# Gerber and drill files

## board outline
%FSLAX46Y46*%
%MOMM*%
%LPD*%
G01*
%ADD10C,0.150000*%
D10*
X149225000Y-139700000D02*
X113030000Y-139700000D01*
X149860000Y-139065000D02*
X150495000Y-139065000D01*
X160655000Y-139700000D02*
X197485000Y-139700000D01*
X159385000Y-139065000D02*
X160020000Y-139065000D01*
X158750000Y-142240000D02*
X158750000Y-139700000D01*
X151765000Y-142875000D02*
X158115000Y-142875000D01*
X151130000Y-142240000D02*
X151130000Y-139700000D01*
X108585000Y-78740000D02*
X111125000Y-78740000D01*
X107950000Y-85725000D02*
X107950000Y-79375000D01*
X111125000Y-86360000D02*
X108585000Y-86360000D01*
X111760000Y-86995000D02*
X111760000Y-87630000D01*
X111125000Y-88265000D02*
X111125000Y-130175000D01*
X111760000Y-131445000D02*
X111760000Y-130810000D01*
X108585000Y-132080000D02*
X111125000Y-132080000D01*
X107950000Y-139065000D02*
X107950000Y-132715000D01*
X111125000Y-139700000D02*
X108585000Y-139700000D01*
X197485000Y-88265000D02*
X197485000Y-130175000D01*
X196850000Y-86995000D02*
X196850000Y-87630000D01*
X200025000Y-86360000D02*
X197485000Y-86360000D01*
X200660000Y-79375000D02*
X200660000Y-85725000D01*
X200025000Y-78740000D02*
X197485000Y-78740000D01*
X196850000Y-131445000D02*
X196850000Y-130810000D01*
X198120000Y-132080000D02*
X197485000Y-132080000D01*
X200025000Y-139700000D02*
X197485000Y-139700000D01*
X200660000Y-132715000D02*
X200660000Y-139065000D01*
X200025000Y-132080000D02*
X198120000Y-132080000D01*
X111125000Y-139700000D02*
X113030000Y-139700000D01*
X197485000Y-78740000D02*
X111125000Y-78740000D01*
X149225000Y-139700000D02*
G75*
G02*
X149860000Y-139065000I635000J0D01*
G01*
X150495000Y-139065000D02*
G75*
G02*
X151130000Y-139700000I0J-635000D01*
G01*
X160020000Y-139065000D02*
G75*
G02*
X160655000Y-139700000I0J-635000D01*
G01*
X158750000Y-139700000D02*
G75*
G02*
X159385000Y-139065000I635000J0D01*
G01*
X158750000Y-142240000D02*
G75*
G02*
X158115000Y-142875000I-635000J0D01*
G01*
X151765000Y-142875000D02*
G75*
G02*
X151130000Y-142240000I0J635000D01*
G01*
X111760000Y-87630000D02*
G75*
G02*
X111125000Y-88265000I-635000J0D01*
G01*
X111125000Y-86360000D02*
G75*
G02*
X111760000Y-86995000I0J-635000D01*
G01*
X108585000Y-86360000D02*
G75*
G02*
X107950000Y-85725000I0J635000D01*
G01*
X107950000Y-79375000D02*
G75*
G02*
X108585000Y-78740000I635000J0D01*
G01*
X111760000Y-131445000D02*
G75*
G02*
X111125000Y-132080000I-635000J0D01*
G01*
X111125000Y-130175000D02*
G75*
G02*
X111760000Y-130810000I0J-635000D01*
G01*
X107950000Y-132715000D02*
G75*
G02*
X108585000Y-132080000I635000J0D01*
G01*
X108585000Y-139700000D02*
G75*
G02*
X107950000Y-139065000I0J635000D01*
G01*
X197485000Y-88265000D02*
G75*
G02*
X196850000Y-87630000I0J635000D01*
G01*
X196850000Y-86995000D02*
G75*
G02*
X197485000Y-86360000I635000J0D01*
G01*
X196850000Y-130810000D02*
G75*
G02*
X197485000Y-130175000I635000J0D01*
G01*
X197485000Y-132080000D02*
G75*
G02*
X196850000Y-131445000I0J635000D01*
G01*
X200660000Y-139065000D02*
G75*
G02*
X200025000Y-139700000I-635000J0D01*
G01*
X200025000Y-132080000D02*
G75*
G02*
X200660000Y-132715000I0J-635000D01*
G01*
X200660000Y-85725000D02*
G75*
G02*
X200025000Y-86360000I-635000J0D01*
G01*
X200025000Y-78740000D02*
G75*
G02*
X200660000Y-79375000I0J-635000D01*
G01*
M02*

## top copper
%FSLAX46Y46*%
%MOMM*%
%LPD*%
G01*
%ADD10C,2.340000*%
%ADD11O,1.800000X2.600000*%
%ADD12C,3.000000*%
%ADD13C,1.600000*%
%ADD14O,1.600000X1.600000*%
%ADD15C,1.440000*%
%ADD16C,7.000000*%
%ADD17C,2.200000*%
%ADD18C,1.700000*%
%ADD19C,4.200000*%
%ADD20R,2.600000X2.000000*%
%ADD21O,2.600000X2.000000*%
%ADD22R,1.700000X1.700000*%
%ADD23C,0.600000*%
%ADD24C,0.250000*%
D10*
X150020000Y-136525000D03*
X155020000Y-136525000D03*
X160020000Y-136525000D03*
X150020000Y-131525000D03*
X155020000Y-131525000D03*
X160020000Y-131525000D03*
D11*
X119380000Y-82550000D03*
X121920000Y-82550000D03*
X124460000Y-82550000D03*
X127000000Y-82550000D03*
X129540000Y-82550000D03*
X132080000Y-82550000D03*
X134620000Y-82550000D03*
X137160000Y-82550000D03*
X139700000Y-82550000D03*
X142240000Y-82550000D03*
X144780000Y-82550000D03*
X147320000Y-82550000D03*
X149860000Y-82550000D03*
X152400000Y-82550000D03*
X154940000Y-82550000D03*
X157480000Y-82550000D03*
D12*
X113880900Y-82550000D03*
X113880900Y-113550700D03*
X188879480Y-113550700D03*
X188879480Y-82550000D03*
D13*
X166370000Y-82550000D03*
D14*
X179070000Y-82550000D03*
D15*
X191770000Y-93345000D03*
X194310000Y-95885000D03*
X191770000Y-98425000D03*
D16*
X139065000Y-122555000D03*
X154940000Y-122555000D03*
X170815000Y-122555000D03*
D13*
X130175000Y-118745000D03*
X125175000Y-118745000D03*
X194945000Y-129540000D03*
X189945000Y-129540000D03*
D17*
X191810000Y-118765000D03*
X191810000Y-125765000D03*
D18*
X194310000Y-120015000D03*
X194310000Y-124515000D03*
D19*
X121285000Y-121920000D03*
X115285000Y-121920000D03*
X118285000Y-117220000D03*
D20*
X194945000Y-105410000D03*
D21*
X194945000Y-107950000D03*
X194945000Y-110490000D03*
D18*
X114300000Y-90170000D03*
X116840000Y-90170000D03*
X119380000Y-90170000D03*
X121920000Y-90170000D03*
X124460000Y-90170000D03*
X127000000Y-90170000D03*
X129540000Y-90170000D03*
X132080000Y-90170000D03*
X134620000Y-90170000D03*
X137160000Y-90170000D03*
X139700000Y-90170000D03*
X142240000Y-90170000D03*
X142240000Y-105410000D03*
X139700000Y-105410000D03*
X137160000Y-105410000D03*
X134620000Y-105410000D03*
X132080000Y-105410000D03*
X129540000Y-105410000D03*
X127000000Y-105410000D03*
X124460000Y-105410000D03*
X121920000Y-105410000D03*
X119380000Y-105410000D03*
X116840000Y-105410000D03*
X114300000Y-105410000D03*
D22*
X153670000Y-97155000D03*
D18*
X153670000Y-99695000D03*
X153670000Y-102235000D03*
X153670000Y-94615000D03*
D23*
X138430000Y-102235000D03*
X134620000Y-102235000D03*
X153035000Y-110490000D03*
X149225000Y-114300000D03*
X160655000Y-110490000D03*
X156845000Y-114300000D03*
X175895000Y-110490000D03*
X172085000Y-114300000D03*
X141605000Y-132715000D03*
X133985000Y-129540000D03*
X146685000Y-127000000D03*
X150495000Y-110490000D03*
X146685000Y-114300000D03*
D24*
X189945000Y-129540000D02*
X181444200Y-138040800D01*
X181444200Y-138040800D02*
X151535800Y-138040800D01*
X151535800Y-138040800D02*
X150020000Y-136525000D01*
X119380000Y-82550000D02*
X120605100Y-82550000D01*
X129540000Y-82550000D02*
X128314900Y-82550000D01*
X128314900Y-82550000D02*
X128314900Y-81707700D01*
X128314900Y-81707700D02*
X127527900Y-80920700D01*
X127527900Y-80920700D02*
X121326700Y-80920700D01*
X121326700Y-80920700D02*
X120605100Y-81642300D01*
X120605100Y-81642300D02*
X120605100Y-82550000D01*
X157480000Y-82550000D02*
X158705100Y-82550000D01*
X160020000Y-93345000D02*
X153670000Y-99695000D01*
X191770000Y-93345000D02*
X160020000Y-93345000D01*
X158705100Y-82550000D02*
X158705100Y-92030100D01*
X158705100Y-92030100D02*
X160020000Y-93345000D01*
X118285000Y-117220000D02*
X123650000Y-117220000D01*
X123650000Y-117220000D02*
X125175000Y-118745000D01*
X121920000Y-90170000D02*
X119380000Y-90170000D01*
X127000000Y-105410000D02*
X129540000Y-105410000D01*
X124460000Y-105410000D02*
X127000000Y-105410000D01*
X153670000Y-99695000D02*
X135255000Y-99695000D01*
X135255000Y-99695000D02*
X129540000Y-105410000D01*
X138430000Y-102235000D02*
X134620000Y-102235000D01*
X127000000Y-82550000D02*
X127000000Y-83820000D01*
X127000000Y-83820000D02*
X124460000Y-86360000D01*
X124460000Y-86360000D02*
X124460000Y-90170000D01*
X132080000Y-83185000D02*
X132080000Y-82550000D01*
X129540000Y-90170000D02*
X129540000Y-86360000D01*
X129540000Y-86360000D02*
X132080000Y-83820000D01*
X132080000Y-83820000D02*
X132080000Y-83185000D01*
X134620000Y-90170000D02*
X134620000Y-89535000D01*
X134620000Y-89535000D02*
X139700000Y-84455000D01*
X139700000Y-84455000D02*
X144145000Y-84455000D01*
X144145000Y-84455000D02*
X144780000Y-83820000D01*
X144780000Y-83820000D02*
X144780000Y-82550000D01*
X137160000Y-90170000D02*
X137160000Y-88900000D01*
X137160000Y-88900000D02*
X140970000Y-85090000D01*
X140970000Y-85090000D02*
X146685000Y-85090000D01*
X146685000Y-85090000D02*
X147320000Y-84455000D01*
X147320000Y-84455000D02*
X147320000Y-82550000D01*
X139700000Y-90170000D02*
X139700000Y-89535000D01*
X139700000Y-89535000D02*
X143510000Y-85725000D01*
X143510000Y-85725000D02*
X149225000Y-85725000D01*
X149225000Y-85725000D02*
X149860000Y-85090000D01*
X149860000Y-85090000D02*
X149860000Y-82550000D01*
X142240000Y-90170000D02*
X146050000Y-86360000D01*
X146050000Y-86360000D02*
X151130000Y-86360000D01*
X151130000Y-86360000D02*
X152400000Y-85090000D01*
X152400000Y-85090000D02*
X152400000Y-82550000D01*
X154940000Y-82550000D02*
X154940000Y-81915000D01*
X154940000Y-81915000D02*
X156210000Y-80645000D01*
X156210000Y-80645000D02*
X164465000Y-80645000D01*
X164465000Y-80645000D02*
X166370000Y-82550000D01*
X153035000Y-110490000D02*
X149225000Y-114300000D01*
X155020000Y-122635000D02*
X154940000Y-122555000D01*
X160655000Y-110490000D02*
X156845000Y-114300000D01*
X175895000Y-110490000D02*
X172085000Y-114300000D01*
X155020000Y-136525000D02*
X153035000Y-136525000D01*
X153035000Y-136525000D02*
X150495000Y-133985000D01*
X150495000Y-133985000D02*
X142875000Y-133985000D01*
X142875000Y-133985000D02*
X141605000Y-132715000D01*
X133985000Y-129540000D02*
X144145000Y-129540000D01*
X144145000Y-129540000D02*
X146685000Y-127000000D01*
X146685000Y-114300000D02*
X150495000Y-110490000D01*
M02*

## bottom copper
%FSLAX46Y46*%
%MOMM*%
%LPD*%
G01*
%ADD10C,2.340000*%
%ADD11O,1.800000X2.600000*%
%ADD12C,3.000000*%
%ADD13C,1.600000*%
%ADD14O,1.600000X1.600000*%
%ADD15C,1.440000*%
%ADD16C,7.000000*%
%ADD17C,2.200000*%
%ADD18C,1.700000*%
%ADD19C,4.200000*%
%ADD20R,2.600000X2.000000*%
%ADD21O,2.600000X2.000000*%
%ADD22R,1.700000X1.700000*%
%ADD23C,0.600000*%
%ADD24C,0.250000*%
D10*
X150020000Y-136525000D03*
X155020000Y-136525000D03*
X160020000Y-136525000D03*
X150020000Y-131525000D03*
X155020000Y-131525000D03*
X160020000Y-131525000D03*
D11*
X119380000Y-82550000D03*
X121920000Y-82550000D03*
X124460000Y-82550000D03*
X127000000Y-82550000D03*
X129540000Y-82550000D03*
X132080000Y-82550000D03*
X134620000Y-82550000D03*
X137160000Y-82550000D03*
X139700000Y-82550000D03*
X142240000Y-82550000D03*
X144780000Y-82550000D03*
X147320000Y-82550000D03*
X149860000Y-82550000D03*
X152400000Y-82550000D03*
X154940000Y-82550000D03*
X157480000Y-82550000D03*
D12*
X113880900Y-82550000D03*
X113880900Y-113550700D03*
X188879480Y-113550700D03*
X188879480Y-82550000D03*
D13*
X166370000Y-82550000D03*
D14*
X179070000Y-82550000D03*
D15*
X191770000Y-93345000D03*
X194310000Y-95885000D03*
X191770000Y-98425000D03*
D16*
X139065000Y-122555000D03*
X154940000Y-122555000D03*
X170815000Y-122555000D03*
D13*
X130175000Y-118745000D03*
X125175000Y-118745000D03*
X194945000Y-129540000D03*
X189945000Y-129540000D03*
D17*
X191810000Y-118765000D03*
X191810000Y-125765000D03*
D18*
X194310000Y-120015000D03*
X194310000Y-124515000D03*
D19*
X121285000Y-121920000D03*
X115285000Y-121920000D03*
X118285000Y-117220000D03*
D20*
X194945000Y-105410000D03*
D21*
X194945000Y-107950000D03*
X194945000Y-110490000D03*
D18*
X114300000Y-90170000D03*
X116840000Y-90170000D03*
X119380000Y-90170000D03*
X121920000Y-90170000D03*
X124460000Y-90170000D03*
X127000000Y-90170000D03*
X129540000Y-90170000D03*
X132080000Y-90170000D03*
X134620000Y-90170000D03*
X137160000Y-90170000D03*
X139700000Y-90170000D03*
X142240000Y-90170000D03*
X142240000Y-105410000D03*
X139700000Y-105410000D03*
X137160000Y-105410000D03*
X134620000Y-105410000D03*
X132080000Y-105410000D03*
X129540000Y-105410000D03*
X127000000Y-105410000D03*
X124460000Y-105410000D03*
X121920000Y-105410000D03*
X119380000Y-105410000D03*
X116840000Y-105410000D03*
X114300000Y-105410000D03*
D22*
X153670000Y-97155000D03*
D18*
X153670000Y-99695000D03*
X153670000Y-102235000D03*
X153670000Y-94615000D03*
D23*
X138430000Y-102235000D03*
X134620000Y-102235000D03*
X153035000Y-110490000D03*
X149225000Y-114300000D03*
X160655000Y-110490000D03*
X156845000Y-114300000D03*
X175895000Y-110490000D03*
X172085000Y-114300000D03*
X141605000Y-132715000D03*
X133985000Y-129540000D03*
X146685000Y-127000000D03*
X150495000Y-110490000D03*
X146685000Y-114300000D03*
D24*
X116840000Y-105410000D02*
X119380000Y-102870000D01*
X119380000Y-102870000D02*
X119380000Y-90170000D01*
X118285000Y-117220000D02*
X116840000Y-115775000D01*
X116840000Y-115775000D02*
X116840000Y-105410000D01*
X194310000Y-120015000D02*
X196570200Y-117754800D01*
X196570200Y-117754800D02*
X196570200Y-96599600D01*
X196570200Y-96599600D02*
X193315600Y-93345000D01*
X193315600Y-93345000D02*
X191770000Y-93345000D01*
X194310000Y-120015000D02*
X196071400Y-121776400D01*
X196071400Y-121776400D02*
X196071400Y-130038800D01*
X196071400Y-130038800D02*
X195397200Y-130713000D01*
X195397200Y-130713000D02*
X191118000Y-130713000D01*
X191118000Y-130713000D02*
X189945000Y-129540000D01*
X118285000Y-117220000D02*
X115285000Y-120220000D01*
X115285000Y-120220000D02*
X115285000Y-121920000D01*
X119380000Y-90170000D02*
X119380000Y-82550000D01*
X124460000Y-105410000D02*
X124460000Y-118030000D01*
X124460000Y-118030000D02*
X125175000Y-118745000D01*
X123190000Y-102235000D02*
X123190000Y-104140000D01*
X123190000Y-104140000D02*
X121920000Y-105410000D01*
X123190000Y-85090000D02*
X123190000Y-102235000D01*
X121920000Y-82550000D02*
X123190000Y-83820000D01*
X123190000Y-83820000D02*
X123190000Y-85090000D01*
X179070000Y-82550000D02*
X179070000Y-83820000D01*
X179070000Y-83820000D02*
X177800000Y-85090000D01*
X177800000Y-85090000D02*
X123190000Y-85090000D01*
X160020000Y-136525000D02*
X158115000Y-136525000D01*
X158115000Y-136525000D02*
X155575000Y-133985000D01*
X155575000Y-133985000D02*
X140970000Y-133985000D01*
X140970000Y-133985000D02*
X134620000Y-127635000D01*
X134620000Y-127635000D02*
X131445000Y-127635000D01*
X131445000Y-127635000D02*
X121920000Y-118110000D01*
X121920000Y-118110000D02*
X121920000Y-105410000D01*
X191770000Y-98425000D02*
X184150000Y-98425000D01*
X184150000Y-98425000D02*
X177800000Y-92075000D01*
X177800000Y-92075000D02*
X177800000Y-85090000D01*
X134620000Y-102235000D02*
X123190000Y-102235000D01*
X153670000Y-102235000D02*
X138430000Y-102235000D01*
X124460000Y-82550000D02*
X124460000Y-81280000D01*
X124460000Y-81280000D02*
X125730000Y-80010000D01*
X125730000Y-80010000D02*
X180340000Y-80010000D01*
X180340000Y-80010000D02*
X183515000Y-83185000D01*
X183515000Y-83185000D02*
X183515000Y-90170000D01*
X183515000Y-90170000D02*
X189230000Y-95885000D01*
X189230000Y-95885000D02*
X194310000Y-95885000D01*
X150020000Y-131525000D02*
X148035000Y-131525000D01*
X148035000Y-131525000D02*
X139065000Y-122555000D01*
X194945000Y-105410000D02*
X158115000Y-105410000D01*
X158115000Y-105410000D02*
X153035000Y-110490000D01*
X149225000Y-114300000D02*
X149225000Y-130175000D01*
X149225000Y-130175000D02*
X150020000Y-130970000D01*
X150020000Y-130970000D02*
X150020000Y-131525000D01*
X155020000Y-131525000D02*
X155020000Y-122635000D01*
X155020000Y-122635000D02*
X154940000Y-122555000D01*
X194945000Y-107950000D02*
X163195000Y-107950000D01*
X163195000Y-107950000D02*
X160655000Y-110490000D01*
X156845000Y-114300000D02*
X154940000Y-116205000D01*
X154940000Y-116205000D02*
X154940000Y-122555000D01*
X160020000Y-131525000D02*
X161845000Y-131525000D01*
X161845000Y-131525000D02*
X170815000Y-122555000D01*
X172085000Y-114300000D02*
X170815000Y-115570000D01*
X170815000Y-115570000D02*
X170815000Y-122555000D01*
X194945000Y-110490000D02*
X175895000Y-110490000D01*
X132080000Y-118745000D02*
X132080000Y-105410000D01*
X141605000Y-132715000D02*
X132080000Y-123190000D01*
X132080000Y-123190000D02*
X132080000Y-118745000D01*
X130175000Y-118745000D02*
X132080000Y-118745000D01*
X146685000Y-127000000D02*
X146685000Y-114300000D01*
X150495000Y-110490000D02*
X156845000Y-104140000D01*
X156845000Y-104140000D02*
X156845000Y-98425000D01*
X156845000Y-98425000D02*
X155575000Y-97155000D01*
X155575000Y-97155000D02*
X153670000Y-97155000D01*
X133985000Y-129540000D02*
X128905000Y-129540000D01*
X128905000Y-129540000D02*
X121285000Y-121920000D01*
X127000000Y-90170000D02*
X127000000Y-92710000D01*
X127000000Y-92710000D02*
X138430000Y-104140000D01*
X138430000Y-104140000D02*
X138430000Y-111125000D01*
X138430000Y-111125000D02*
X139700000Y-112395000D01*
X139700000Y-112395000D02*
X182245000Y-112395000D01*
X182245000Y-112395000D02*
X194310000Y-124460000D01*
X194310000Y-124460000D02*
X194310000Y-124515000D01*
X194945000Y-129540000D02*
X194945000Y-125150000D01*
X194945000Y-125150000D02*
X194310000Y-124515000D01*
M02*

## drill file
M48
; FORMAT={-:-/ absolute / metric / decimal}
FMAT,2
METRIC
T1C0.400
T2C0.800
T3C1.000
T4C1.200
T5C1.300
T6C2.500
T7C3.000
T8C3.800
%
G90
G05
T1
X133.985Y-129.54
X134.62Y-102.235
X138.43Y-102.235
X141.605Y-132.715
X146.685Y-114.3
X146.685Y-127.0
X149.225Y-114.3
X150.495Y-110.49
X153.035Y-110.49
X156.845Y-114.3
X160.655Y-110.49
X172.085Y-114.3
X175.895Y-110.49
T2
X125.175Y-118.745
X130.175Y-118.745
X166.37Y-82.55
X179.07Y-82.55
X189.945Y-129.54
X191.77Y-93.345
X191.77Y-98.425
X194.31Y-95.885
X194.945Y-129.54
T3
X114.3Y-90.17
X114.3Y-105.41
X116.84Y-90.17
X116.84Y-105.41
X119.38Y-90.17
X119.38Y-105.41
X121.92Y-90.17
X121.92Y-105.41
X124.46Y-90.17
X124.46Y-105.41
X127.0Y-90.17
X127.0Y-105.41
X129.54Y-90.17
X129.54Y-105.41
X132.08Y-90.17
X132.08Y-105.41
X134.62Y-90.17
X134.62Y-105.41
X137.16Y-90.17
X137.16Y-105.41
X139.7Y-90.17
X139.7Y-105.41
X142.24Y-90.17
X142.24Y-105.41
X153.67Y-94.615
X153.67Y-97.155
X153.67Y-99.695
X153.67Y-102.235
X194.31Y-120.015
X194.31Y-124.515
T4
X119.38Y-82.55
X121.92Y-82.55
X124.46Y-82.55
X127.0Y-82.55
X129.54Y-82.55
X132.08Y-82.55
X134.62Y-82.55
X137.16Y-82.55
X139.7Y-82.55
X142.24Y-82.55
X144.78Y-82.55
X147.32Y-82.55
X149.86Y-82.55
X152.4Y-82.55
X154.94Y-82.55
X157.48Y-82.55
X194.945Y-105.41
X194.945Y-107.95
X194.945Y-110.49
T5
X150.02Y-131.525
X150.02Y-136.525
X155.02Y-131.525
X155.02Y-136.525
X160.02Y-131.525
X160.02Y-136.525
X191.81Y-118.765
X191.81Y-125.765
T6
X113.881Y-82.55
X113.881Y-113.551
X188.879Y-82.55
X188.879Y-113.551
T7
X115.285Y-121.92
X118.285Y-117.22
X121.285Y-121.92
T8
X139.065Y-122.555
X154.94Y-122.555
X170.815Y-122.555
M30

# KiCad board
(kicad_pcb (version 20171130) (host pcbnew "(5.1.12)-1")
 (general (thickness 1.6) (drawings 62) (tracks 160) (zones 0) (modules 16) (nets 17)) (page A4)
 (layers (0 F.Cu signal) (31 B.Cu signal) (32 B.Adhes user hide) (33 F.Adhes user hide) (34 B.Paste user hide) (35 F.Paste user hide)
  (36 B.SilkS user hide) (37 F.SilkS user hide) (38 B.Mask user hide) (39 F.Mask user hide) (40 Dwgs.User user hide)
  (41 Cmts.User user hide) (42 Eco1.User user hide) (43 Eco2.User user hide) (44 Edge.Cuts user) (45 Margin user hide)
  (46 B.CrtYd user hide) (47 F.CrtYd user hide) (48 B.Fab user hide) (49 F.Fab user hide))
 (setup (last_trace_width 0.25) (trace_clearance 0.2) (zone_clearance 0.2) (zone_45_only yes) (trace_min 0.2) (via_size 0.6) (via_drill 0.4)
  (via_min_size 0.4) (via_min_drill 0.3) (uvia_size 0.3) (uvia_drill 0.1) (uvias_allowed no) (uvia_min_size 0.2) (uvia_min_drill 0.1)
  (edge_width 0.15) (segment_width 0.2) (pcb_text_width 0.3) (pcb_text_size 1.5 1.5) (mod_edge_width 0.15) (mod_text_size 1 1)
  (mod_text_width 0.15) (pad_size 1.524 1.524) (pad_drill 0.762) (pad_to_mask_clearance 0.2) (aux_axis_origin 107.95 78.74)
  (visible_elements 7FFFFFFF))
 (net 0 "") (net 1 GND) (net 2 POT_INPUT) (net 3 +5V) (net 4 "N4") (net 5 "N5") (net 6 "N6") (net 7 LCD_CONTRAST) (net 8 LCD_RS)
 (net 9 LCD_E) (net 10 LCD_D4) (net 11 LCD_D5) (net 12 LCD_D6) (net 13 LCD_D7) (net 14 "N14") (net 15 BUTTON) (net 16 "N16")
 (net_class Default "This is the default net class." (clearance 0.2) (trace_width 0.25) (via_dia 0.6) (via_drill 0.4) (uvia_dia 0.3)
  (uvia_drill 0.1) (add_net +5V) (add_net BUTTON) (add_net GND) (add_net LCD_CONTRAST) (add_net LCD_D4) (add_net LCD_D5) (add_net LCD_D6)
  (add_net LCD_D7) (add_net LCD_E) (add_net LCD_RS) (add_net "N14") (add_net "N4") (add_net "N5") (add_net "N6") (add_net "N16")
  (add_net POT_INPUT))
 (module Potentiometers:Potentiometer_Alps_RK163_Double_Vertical (layer B.Cu) (at 160.02 136.525 270)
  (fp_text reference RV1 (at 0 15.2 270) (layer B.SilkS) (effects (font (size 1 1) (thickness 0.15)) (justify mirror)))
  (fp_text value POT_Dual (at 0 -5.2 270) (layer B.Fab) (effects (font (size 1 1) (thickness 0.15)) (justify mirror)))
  (pad 3 thru_hole circle (at 0 10 270) (size 2.34 2.34) (drill 1.3) (layers *.Cu *.Mask) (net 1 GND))
  (pad 2 thru_hole circle (at 0 5 270) (size 2.34 2.34) (drill 1.3) (layers *.Cu *.Mask) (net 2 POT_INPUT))
  (pad 1 thru_hole circle (at 0 0 270) (size 2.34 2.34) (drill 1.3) (layers *.Cu *.Mask) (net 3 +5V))
  (pad 6 thru_hole circle (at -5 10 270) (size 2.34 2.34) (drill 1.3) (layers *.Cu *.Mask) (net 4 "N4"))
  (pad 5 thru_hole circle (at -5 5 270) (size 2.34 2.34) (drill 1.3) (layers *.Cu *.Mask) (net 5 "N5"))
  (pad 4 thru_hole circle (at -5 0 270) (size 2.34 2.34) (drill 1.3) (layers *.Cu *.Mask) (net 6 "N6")))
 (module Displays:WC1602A (layer F.Cu) (at 119.38 82.55)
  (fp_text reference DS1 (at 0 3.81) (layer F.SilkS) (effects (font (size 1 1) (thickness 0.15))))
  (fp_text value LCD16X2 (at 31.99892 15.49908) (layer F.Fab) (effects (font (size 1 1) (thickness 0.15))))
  (pad 1 thru_hole oval (at 0 0) (size 1.8 2.6) (drill 1.2) (layers *.Cu *.Mask) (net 1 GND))
  (pad 2 thru_hole oval (at 2.54 0) (size 1.8 2.6) (drill 1.2) (layers *.Cu *.Mask) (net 3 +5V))
  (pad 3 thru_hole oval (at 5.08 0) (size 1.8 2.6) (drill 1.2) (layers *.Cu *.Mask) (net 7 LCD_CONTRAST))
  (pad 4 thru_hole oval (at 7.62 0) (size 1.8 2.6) (drill 1.2) (layers *.Cu *.Mask) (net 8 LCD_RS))
  (pad 5 thru_hole oval (at 10.16 0) (size 1.8 2.6) (drill 1.2) (layers *.Cu *.Mask) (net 1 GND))
  (pad 6 thru_hole oval (at 12.7 0) (size 1.8 2.6) (drill 1.2) (layers *.Cu *.Mask) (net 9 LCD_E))
  (pad 7 thru_hole oval (at 15.24 0) (size 1.8 2.6) (drill 1.2) (layers *.Cu *.Mask))
  (pad 8 thru_hole oval (at 17.78 0) (size 1.8 2.6) (drill 1.2) (layers *.Cu *.Mask))
  (pad 9 thru_hole oval (at 20.32 0) (size 1.8 2.6) (drill 1.2) (layers *.Cu *.Mask))
  (pad 10 thru_hole oval (at 22.86 0) (size 1.8 2.6) (drill 1.2) (layers *.Cu *.Mask))
  (pad 11 thru_hole oval (at 25.4 0) (size 1.8 2.6) (drill 1.2) (layers *.Cu *.Mask) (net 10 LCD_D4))
  (pad 12 thru_hole oval (at 27.94 0) (size 1.8 2.6) (drill 1.2) (layers *.Cu *.Mask) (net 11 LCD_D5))
  (pad 13 thru_hole oval (at 30.48 0) (size 1.8 2.6) (drill 1.2) (layers *.Cu *.Mask) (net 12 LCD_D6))
  (pad 14 thru_hole oval (at 33.02 0) (size 1.8 2.6) (drill 1.2) (layers *.Cu *.Mask) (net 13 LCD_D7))
  (pad 15 thru_hole oval (at 35.56 0) (size 1.8 2.6) (drill 1.2) (layers *.Cu *.Mask) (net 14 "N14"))
  (pad 16 thru_hole oval (at 38.1 0) (size 1.8 2.6) (drill 1.2) (layers *.Cu *.Mask) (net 1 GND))
  (pad 0 thru_hole circle (at -5.4991 0) (size 3 3) (drill 2.5) (layers *.Cu *.Mask))
  (pad 0 thru_hole circle (at -5.4991 31.0007) (size 3 3) (drill 2.5) (layers *.Cu *.Mask))
  (pad 0 thru_hole circle (at 69.49948 31.0007) (size 3 3) (drill 2.5) (layers *.Cu *.Mask))
  (pad 0 thru_hole circle (at 69.49948 0) (size 3 3) (drill 2.5) (layers *.Cu *.Mask)))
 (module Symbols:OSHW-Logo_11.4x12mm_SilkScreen (layer F.Cu) (at 182.245 124.46)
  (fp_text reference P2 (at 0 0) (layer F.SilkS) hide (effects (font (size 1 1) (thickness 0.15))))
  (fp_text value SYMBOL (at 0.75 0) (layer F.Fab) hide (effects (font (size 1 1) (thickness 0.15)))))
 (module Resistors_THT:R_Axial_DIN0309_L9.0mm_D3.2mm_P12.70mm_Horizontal (layer B.Cu) (at 166.37 82.55)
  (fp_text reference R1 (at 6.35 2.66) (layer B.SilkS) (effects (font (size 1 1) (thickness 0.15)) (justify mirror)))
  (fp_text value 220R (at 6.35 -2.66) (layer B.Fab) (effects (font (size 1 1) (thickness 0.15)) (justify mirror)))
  (pad 1 thru_hole circle (at 0 0) (size 1.6 1.6) (drill 0.8) (layers *.Cu *.Mask) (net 14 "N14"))
  (pad 2 thru_hole oval (at 12.7 0) (size 1.6 1.6) (drill 0.8) (layers *.Cu *.Mask) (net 3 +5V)))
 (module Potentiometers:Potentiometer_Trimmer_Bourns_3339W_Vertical (layer B.Cu) (at 191.77 98.425)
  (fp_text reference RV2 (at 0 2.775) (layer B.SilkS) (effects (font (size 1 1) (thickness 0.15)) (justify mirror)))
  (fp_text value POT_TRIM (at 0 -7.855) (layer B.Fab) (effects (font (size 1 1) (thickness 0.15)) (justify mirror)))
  (pad 3 thru_hole circle (at 0 -5.08) (size 1.44 1.44) (drill 0.8) (layers *.Cu *.Mask) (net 1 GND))
  (pad 2 thru_hole circle (at 2.54 -2.54) (size 1.44 1.44) (drill 0.8) (layers *.Cu *.Mask) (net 7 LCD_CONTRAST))
  (pad 1 thru_hole circle (at 0 0) (size 1.44 1.44) (drill 0.8) (layers *.Cu *.Mask) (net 3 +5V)))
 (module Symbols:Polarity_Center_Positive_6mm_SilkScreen (layer F.Cu) (at 127 132.715)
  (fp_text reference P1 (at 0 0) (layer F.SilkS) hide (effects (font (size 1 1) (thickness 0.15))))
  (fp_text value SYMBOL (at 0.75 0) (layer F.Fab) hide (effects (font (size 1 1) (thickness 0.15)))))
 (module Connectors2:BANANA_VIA (layer F.Cu) (at 139.065 122.555)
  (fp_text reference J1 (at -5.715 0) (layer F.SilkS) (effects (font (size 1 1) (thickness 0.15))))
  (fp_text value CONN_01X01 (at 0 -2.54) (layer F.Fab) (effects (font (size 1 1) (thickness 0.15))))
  (pad 1 thru_hole circle (at 0 0) (size 7 7) (drill 3.8) (layers *.Cu *.Mask) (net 4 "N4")))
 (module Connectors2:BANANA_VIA (layer F.Cu) (at 154.94 122.555)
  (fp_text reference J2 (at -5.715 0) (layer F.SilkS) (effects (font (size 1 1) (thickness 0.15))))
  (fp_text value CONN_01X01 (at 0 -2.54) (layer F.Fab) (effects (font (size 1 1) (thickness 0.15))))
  (pad 1 thru_hole circle (at 0 0) (size 7 7) (drill 3.8) (layers *.Cu *.Mask) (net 5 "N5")))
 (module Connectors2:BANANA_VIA (layer F.Cu) (at 170.815 122.555)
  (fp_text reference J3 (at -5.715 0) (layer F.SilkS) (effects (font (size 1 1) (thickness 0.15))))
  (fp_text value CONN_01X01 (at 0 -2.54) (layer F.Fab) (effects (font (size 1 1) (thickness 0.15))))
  (pad 1 thru_hole circle (at 0 0) (size 7 7) (drill 3.8) (layers *.Cu *.Mask) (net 6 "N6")))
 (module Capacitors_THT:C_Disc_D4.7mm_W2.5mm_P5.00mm (layer B.Cu) (at 130.175 118.745 180)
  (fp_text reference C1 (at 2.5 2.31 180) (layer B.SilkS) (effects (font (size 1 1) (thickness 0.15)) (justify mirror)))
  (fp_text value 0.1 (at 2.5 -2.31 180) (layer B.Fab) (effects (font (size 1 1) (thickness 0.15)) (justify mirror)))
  (pad 1 thru_hole circle (at 0 0 180) (size 1.6 1.6) (drill 0.8) (layers *.Cu *.Mask) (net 2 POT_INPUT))
  (pad 2 thru_hole circle (at 5 0 180) (size 1.6 1.6) (drill 0.8) (layers *.Cu *.Mask) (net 1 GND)))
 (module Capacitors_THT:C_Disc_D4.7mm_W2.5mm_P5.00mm (layer B.Cu) (at 194.945 129.54 180)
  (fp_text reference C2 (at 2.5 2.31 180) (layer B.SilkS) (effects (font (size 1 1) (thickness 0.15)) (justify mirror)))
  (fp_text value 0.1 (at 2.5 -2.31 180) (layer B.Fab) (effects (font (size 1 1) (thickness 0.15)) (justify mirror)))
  (pad 1 thru_hole circle (at 0 0 180) (size 1.6 1.6) (drill 0.8) (layers *.Cu *.Mask) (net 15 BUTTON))
  (pad 2 thru_hole circle (at 5 0 180) (size 1.6 1.6) (drill 0.8) (layers *.Cu *.Mask) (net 1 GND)))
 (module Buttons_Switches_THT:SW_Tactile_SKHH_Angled (layer B.Cu) (at 194.31 120.015 270)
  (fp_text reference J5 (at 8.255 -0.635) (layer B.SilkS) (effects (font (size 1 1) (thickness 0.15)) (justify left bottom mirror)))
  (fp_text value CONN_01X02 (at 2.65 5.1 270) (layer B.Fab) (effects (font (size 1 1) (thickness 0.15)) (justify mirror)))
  (pad "" thru_hole circle (at -1.25 2.5 270) (size 2.2 2.2) (drill 1.3) (layers *.Cu *.Mask))
  (pad "" thru_hole circle (at 5.75 2.5 270) (size 2.2 2.2) (drill 1.3) (layers *.Cu *.Mask))
  (pad 1 thru_hole circle (at 0 0 270) (size 1.7 1.7) (drill 1) (layers *.Cu *.Mask) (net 1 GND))
  (pad 2 thru_hole circle (at 4.5 0 270) (size 1.7 1.7) (drill 1) (layers *.Cu *.Mask) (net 15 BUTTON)))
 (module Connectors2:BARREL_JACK (layer B.Cu) (at 121.285 121.92)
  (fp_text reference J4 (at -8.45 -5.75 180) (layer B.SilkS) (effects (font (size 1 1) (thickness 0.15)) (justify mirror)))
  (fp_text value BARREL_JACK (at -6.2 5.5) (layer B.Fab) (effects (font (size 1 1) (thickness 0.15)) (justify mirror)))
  (pad 1 thru_hole circle (at 0 0) (size 4.2 4.2) (drill 3) (layers *.Cu *.Mask) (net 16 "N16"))
  (pad 2 thru_hole circle (at -6 0) (size 4.2 4.2) (drill 3) (layers *.Cu *.Mask) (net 1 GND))
  (pad 3 thru_hole circle (at -3 -4.7) (size 4.2 4.2) (drill 3) (layers *.Cu *.Mask) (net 1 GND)))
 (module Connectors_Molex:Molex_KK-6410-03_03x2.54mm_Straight (layer F.Cu) (at 194.945 105.41 270)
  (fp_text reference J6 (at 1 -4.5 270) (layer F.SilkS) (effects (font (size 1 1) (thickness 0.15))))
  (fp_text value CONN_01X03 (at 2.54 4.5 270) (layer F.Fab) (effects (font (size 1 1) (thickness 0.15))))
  (pad 1 thru_hole rect (at 0 0 270) (size 2 2.6) (drill 1.2) (layers *.Cu *.Mask) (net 4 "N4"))
  (pad 2 thru_hole oval (at 2.54 0 270) (size 2 2.6) (drill 1.2) (layers *.Cu *.Mask) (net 5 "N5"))
  (pad 3 thru_hole oval (at 5.08 0 270) (size 2 2.6) (drill 1.2) (layers *.Cu *.Mask) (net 6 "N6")))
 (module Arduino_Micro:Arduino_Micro (layer B.Cu) (at 128.27 97.79 270)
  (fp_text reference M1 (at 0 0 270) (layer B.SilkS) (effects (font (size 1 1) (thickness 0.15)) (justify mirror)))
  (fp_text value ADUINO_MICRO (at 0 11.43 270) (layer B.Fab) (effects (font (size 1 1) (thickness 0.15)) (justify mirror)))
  (pad 1 thru_hole circle (at -7.62 13.97 270) (size 1.7 1.7) (drill 1) (layers *.Cu *.Mask))
  (pad 2 thru_hole circle (at -7.62 11.43 270) (size 1.7 1.7) (drill 1) (layers *.Cu *.Mask))
  (pad 3 thru_hole circle (at -7.62 8.89 270) (size 1.7 1.7) (drill 1) (layers *.Cu *.Mask) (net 1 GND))
  (pad 4 thru_hole circle (at -7.62 6.35 270) (size 1.7 1.7) (drill 1) (layers *.Cu *.Mask) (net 1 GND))
  (pad 5 thru_hole circle (at -7.62 3.81 270) (size 1.7 1.7) (drill 1) (layers *.Cu *.Mask) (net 8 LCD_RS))
  (pad 6 thru_hole circle (at -7.62 1.27 270) (size 1.7 1.7) (drill 1) (layers *.Cu *.Mask) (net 15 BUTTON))
  (pad 7 thru_hole circle (at -7.62 -1.27 270) (size 1.7 1.7) (drill 1) (layers *.Cu *.Mask) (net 9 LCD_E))
  (pad 8 thru_hole circle (at -7.62 -3.81 270) (size 1.7 1.7) (drill 1) (layers *.Cu *.Mask))
  (pad 9 thru_hole circle (at -7.62 -6.35 270) (size 1.7 1.7) (drill 1) (layers *.Cu *.Mask) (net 10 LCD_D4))
  (pad 10 thru_hole circle (at -7.62 -8.89 270) (size 1.7 1.7) (drill 1) (layers *.Cu *.Mask) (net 11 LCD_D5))
  (pad 11 thru_hole circle (at -7.62 -11.43 270) (size 1.7 1.7) (drill 1) (layers *.Cu *.Mask) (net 12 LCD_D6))
  (pad 12 thru_hole circle (at -7.62 -13.97 270) (size 1.7 1.7) (drill 1) (layers *.Cu *.Mask) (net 13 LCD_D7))
  (pad 13 thru_hole circle (at 7.62 -13.97 270) (size 1.7 1.7) (drill 1) (layers *.Cu *.Mask))
  (pad 14 thru_hole circle (at 7.62 -11.43 270) (size 1.7 1.7) (drill 1) (layers *.Cu *.Mask))
  (pad 15 thru_hole circle (at 7.62 -8.89 270) (size 1.7 1.7) (drill 1) (layers *.Cu *.Mask))
  (pad 16 thru_hole circle (at 7.62 -6.35 270) (size 1.7 1.7) (drill 1) (layers *.Cu *.Mask))
  (pad 17 thru_hole circle (at 7.62 -3.81 270) (size 1.7 1.7) (drill 1) (layers *.Cu *.Mask) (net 2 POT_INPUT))
  (pad 18 thru_hole circle (at 7.62 -1.27 270) (size 1.7 1.7) (drill 1) (layers *.Cu *.Mask) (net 1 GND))
  (pad 19 thru_hole circle (at 7.62 1.27 270) (size 1.7 1.7) (drill 1) (layers *.Cu *.Mask) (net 1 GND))
  (pad 20 thru_hole circle (at 7.62 3.81 270) (size 1.7 1.7) (drill 1) (layers *.Cu *.Mask) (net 1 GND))
  (pad 21 thru_hole circle (at 7.62 6.35 270) (size 1.7 1.7) (drill 1) (layers *.Cu *.Mask) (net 3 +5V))
  (pad 22 thru_hole circle (at 7.62 8.89 270) (size 1.7 1.7) (drill 1) (layers *.Cu *.Mask))
  (pad 23 thru_hole circle (at 7.62 11.43 270) (size 1.7 1.7) (drill 1) (layers *.Cu *.Mask) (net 1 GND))
  (pad 24 thru_hole circle (at 7.62 13.97 270) (size 1.7 1.7) (drill 1) (layers *.Cu *.Mask)))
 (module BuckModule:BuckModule (layer B.Cu) (at 153.67 99.695 270)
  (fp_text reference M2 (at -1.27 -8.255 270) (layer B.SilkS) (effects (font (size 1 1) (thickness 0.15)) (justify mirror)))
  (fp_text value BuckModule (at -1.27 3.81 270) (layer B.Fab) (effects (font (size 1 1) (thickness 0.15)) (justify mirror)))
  (pad 1 thru_hole rect (at -2.54 0 270) (size 1.7 1.7) (drill 1) (layers *.Cu *.Mask) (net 16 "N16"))
  (pad 2 thru_hole circle (at 0 0 270) (size 1.7 1.7) (drill 1) (layers *.Cu *.Mask) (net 1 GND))
  (pad 3 thru_hole circle (at 2.54 0 270) (size 1.7 1.7) (drill 1) (layers *.Cu *.Mask) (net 3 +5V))
  (pad 4 thru_hole circle (at -5.08 0 270) (size 1.7 1.7) (drill 1) (layers *.Cu *.Mask)))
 (gr_line (start 149.225 139.7) (end 113.03 139.7) (angle 90) (layer Edge.Cuts) (width 0.15))
 (gr_line (start 149.86 139.065) (end 150.495 139.065) (angle 90) (layer Edge.Cuts) (width 0.15))
 (gr_line (start 160.655 139.7) (end 197.485 139.7) (angle 90) (layer Edge.Cuts) (width 0.15))
 (gr_line (start 159.385 139.065) (end 160.02 139.065) (angle 90) (layer Edge.Cuts) (width 0.15))
 (gr_line (start 158.75 142.24) (end 158.75 139.7) (angle 90) (layer Edge.Cuts) (width 0.15))
 (gr_line (start 151.765 142.875) (end 158.115 142.875) (angle 90) (layer Edge.Cuts) (width 0.15))
 (gr_line (start 151.13 142.24) (end 151.13 139.7) (angle 90) (layer Edge.Cuts) (width 0.15))
 (gr_line (start 108.585 78.74) (end 111.125 78.74) (angle 90) (layer Edge.Cuts) (width 0.15))
 (gr_line (start 107.95 85.725) (end 107.95 79.375) (angle 90) (layer Edge.Cuts) (width 0.15))
 (gr_line (start 111.125 86.36) (end 108.585 86.36) (angle 90) (layer Edge.Cuts) (width 0.15))
 (gr_line (start 111.76 86.995) (end 111.76 87.63) (angle 90) (layer Edge.Cuts) (width 0.15))
 (gr_line (start 111.125 88.265) (end 111.125 130.175) (angle 90) (layer Edge.Cuts) (width 0.15))
 (gr_line (start 111.76 131.445) (end 111.76 130.81) (angle 90) (layer Edge.Cuts) (width 0.15))
 (gr_line (start 108.585 132.08) (end 111.125 132.08) (angle 90) (layer Edge.Cuts) (width 0.15))
 (gr_line (start 107.95 139.065) (end 107.95 132.715) (angle 90) (layer Edge.Cuts) (width 0.15))
 (gr_line (start 111.125 139.7) (end 108.585 139.7) (angle 90) (layer Edge.Cuts) (width 0.15))
 (gr_line (start 197.485 88.265) (end 197.485 130.175) (angle 90) (layer Edge.Cuts) (width 0.15))
 (gr_line (start 196.85 86.995) (end 196.85 87.63) (angle 90) (layer Edge.Cuts) (width 0.15))
 (gr_line (start 200.025 86.36) (end 197.485 86.36) (angle 90) (layer Edge.Cuts) (width 0.15))
 (gr_line (start 200.66 79.375) (end 200.66 85.725) (angle 90) (layer Edge.Cuts) (width 0.15))
 (gr_line (start 200.025 78.74) (end 197.485 78.74) (angle 90) (layer Edge.Cuts) (width 0.15))
 (gr_line (start 196.85 131.445) (end 196.85 130.81) (angle 90) (layer Edge.Cuts) (width 0.15))
 (gr_line (start 198.12 132.08) (end 197.485 132.08) (angle 90) (layer Edge.Cuts) (width 0.15))
 (gr_line (start 200.025 139.7) (end 197.485 139.7) (angle 90) (layer Edge.Cuts) (width 0.15))
 (gr_line (start 200.66 132.715) (end 200.66 139.065) (angle 90) (layer Edge.Cuts) (width 0.15))
 (gr_line (start 200.025 132.08) (end 198.12 132.08) (angle 90) (layer Edge.Cuts) (width 0.15))
 (gr_line (start 111.125 139.7) (end 113.03 139.7) (angle 90) (layer Edge.Cuts) (width 0.15))
 (gr_line (start 197.485 78.74) (end 111.125 78.74) (angle 90) (layer Edge.Cuts) (width 0.15))
 (gr_arc (start 149.86 139.7) (end 149.225 139.7) (angle 90) (layer Edge.Cuts) (width 0.15))
 (gr_arc (start 150.495 139.7) (end 150.495 139.065) (angle 90) (layer Edge.Cuts) (width 0.15))
 (gr_arc (start 160.02 139.7) (end 160.02 139.065) (angle 90) (layer Edge.Cuts) (width 0.15))
 (gr_arc (start 159.385 139.7) (end 158.75 139.7) (angle 90) (layer Edge.Cuts) (width 0.15))
 (gr_arc (start 158.115 142.24) (end 158.75 142.24) (angle 90) (layer Edge.Cuts) (width 0.15))
 (gr_arc (start 151.765 142.24) (end 151.765 142.875) (angle 90) (layer Edge.Cuts) (width 0.15))
 (gr_arc (start 111.125 87.63) (end 111.76 87.63) (angle 90) (layer Edge.Cuts) (width 0.15))
 (gr_arc (start 111.125 86.995) (end 111.125 86.36) (angle 90) (layer Edge.Cuts) (width 0.15))
 (gr_arc (start 108.585 85.725) (end 108.585 86.36) (angle 90) (layer Edge.Cuts) (width 0.15))
 (gr_arc (start 108.585 79.375) (end 107.95 79.375) (angle 90) (layer Edge.Cuts) (width 0.15))
 (gr_arc (start 111.125 131.445) (end 111.76 131.445) (angle 90) (layer Edge.Cuts) (width 0.15))
 (gr_arc (start 111.125 130.81) (end 111.125 130.175) (angle 90) (layer Edge.Cuts) (width 0.15))
 (gr_arc (start 108.585 132.715) (end 107.95 132.715) (angle 90) (layer Edge.Cuts) (width 0.15))
 (gr_arc (start 108.585 139.065) (end 108.585 139.7) (angle 90) (layer Edge.Cuts) (width 0.15))
 (gr_arc (start 197.485 87.63) (end 197.485 88.265) (angle 90) (layer Edge.Cuts) (width 0.15))
 (gr_arc (start 197.485 86.995) (end 196.85 86.995) (angle 90) (layer Edge.Cuts) (width 0.15))
 (gr_arc (start 197.485 130.81) (end 196.85 130.81) (angle 90) (layer Edge.Cuts) (width 0.15))
 (gr_arc (start 197.485 131.445) (end 197.485 132.08) (angle 90) (layer Edge.Cuts) (width 0.15))
 (gr_arc (start 200.025 139.065) (end 200.66 139.065) (angle 90) (layer Edge.Cuts) (width 0.15))
 (gr_arc (start 200.025 132.715) (end 200.025 132.08) (angle 90) (layer Edge.Cuts) (width 0.15))
 (gr_arc (start 200.025 85.725) (end 200.66 85.725) (angle 90) (layer Edge.Cuts) (width 0.15))
 (gr_arc (start 200.025 79.375) (end 200.025 78.74) (angle 90) (layer Edge.Cuts) (width 0.15))
 (segment (start 189.945 129.54) (end 181.4442 138.0408) (width 0.25) (layer F.Cu) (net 1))
 (segment (start 181.4442 138.0408) (end 151.5358 138.0408) (width 0.25) (layer F.Cu) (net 1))
 (segment (start 151.5358 138.0408) (end 150.02 136.525) (width 0.25) (layer F.Cu) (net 1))
 (segment (start 119.38 82.55) (end 120.6051 82.55) (width 0.25) (layer F.Cu) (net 1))
 (segment (start 129.54 82.55) (end 128.3149 82.55) (width 0.25) (layer F.Cu) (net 1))
 (segment (start 128.3149 82.55) (end 128.3149 81.7077) (width 0.25) (layer F.Cu) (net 1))
 (segment (start 128.3149 81.7077) (end 127.5279 80.9207) (width 0.25) (layer F.Cu) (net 1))
 (segment (start 127.5279 80.9207) (end 121.3267 80.9207) (width 0.25) (layer F.Cu) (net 1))
 (segment (start 121.3267 80.9207) (end 120.6051 81.6423) (width 0.25) (layer F.Cu) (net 1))
 (segment (start 120.6051 81.6423) (end 120.6051 82.55) (width 0.25) (layer F.Cu) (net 1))
 (segment (start 157.48 82.55) (end 158.7051 82.55) (width 0.25) (layer F.Cu) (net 1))
 (segment (start 160.02 93.345) (end 153.67 99.695) (width 0.25) (layer F.Cu) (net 1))
 (segment (start 191.77 93.345) (end 160.02 93.345) (width 0.25) (layer F.Cu) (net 1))
 (segment (start 158.7051 82.55) (end 158.7051 92.0301) (width 0.25) (layer F.Cu) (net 1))
 (segment (start 158.7051 92.0301) (end 160.02 93.345) (width 0.25) (layer F.Cu) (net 1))
 (segment (start 116.84 105.41) (end 119.38 102.87) (width 0.25) (layer B.Cu) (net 1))
 (segment (start 119.38 102.87) (end 119.38 90.17) (width 0.25) (layer B.Cu) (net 1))
 (segment (start 118.285 117.22) (end 116.84 115.775) (width 0.25) (layer B.Cu) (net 1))
 (segment (start 116.84 115.775) (end 116.84 105.41) (width 0.25) (layer B.Cu) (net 1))
 (segment (start 194.31 120.015) (end 196.5702 117.7548) (width 0.25) (layer B.Cu) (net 1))
 (segment (start 196.5702 117.7548) (end 196.5702 96.5996) (width 0.25) (layer B.Cu) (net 1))
 (segment (start 196.5702 96.5996) (end 193.3156 93.345) (width 0.25) (layer B.Cu) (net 1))
 (segment (start 193.3156 93.345) (end 191.77 93.345) (width 0.25) (layer B.Cu) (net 1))
 (segment (start 194.31 120.015) (end 196.0714 121.7764) (width 0.25) (layer B.Cu) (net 1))
 (segment (start 196.0714 121.7764) (end 196.0714 130.0388) (width 0.25) (layer B.Cu) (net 1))
 (segment (start 196.0714 130.0388) (end 195.3972 130.713) (width 0.25) (layer B.Cu) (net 1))
 (segment (start 195.3972 130.713) (end 191.118 130.713) (width 0.25) (layer B.Cu) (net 1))
 (segment (start 191.118 130.713) (end 189.945 129.54) (width 0.25) (layer B.Cu) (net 1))
 (segment (start 118.285 117.22) (end 123.65 117.22) (width 0.25) (layer F.Cu) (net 1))
 (segment (start 123.65 117.22) (end 125.175 118.745) (width 0.25) (layer F.Cu) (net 1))
 (segment (start 118.285 117.22) (end 115.285 120.22) (width 0.25) (layer B.Cu) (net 1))
 (segment (start 115.285 120.22) (end 115.285 121.92) (width 0.25) (layer B.Cu) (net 1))
 (segment (start 119.38 90.17) (end 119.38 82.55) (width 0.25) (layer B.Cu) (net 1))
 (segment (start 121.92 90.17) (end 119.38 90.17) (width 0.25) (layer F.Cu) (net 1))
 (segment (start 124.46 105.41) (end 124.46 118.03) (width 0.25) (layer B.Cu) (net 1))
 (segment (start 124.46 118.03) (end 125.175 118.745) (width 0.25) (layer B.Cu) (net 1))
 (segment (start 127 105.41) (end 129.54 105.41) (width 0.25) (layer F.Cu) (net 1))
 (segment (start 124.46 105.41) (end 127 105.41) (width 0.25) (layer F.Cu) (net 1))
 (segment (start 153.67 99.695) (end 135.255 99.695) (width 0.25) (layer F.Cu) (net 1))
 (segment (start 135.255 99.695) (end 129.54 105.41) (width 0.25) (layer F.Cu) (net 1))
 (segment (start 123.19 102.235) (end 123.19 104.14) (width 0.25) (layer B.Cu) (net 3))
 (segment (start 123.19 104.14) (end 121.92 105.41) (width 0.25) (layer B.Cu) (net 3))
 (segment (start 123.19 85.09) (end 123.19 102.235) (width 0.25) (layer B.Cu) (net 3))
 (segment (start 121.92 82.55) (end 123.19 83.82) (width 0.25) (layer B.Cu) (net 3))
 (segment (start 123.19 83.82) (end 123.19 85.09) (width 0.25) (layer B.Cu) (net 3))
 (segment (start 179.07 82.55) (end 179.07 83.82) (width 0.25) (layer B.Cu) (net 3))
 (segment (start 179.07 83.82) (end 177.8 85.09) (width 0.25) (layer B.Cu) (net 3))
 (segment (start 177.8 85.09) (end 123.19 85.09) (width 0.25) (layer B.Cu) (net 3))
 (segment (start 160.02 136.525) (end 158.115 136.525) (width 0.25) (layer B.Cu) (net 3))
 (segment (start 158.115 136.525) (end 155.575 133.985) (width 0.25) (layer B.Cu) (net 3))
 (segment (start 155.575 133.985) (end 140.97 133.985) (width 0.25) (layer B.Cu) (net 3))
 (segment (start 140.97 133.985) (end 134.62 127.635) (width 0.25) (layer B.Cu) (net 3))
 (segment (start 134.62 127.635) (end 131.445 127.635) (width 0.25) (layer B.Cu) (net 3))
 (segment (start 131.445 127.635) (end 121.92 118.11) (width 0.25) (layer B.Cu) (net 3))
 (segment (start 121.92 118.11) (end 121.92 105.41) (width 0.25) (layer B.Cu) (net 3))
 (segment (start 191.77 98.425) (end 184.15 98.425) (width 0.25) (layer B.Cu) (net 3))
 (segment (start 184.15 98.425) (end 177.8 92.075) (width 0.25) (layer B.Cu) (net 3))
 (segment (start 177.8 92.075) (end 177.8 85.09) (width 0.25) (layer B.Cu) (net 3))
 (segment (start 138.43 102.235) (end 134.62 102.235) (width 0.25) (layer F.Cu) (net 3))
 (segment (start 134.62 102.235) (end 123.19 102.235) (width 0.25) (layer B.Cu) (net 3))
 (segment (start 153.67 102.235) (end 138.43 102.235) (width 0.25) (layer B.Cu) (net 3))
 (via (at 138.43 102.235) (size 0.6) (layers F.Cu B.Cu) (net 3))
 (via (at 134.62 102.235) (size 0.6) (layers F.Cu B.Cu) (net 3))
 (segment (start 124.46 82.55) (end 124.46 81.28) (width 0.25) (layer B.Cu) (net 7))
 (segment (start 124.46 81.28) (end 125.73 80.01) (width 0.25) (layer B.Cu) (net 7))
 (segment (start 125.73 80.01) (end 180.34 80.01) (width 0.25) (layer B.Cu) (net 7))
 (segment (start 180.34 80.01) (end 183.515 83.185) (width 0.25) (layer B.Cu) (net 7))
 (segment (start 183.515 83.185) (end 183.515 90.17) (width 0.25) (layer B.Cu) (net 7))
 (segment (start 183.515 90.17) (end 189.23 95.885) (width 0.25) (layer B.Cu) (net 7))
 (segment (start 189.23 95.885) (end 194.31 95.885) (width 0.25) (layer B.Cu) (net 7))
 (segment (start 127 82.55) (end 127 83.82) (width 0.25) (layer F.Cu) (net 8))
 (segment (start 127 83.82) (end 124.46 86.36) (width 0.25) (layer F.Cu) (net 8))
 (segment (start 124.46 86.36) (end 124.46 90.17) (width 0.25) (layer F.Cu) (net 8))
 (segment (start 132.08 83.185) (end 132.08 82.55) (width 0.25) (layer F.Cu) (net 9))
 (segment (start 129.54 90.17) (end 129.54 86.36) (width 0.25) (layer F.Cu) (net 9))
 (segment (start 129.54 86.36) (end 132.08 83.82) (width 0.25) (layer F.Cu) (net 9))
 (segment (start 132.08 83.82) (end 132.08 83.185) (width 0.25) (layer F.Cu) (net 9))
 (segment (start 134.62 90.17) (end 134.62 89.535) (width 0.25) (layer F.Cu) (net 10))
 (segment (start 134.62 89.535) (end 139.7 84.455) (width 0.25) (layer F.Cu) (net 10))
 (segment (start 139.7 84.455) (end 144.145 84.455) (width 0.25) (layer F.Cu) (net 10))
 (segment (start 144.145 84.455) (end 144.78 83.82) (width 0.25) (layer F.Cu) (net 10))
 (segment (start 144.78 83.82) (end 144.78 82.55) (width 0.25) (layer F.Cu) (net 10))
 (segment (start 137.16 90.17) (end 137.16 88.9) (width 0.25) (layer F.Cu) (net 11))
 (segment (start 137.16 88.9) (end 140.97 85.09) (width 0.25) (layer F.Cu) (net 11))
 (segment (start 140.97 85.09) (end 146.685 85.09) (width 0.25) (layer F.Cu) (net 11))
 (segment (start 146.685 85.09) (end 147.32 84.455) (width 0.25) (layer F.Cu) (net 11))
 (segment (start 147.32 84.455) (end 147.32 82.55) (width 0.25) (layer F.Cu) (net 11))
 (segment (start 139.7 90.17) (end 139.7 89.535) (width 0.25) (layer F.Cu) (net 12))
 (segment (start 139.7 89.535) (end 143.51 85.725) (width 0.25) (layer F.Cu) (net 12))
 (segment (start 143.51 85.725) (end 149.225 85.725) (width 0.25) (layer F.Cu) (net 12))
 (segment (start 149.225 85.725) (end 149.86 85.09) (width 0.25) (layer F.Cu) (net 12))
 (segment (start 149.86 85.09) (end 149.86 82.55) (width 0.25) (layer F.Cu) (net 12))
 (segment (start 142.24 90.17) (end 146.05 86.36) (width 0.25) (layer F.Cu) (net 13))
 (segment (start 146.05 86.36) (end 151.13 86.36) (width 0.25) (layer F.Cu) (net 13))
 (segment (start 151.13 86.36) (end 152.4 85.09) (width 0.25) (layer F.Cu) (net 13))
 (segment (start 152.4 85.09) (end 152.4 82.55) (width 0.25) (layer F.Cu) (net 13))
 (segment (start 154.94 82.55) (end 154.94 81.915) (width 0.25) (layer F.Cu) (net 14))
 (segment (start 154.94 81.915) (end 156.21 80.645) (width 0.25) (layer F.Cu) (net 14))
 (segment (start 156.21 80.645) (end 164.465 80.645) (width 0.25) (layer F.Cu) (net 14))
 (segment (start 164.465 80.645) (end 166.37 82.55) (width 0.25) (layer F.Cu) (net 14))
 (segment (start 150.02 131.525) (end 148.035 131.525) (width 0.25) (layer B.Cu) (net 4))
 (segment (start 148.035 131.525) (end 139.065 122.555) (width 0.25) (layer B.Cu) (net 4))
 (segment (start 194.945 105.41) (end 158.115 105.41) (width 0.25) (layer B.Cu) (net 4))
 (segment (start 158.115 105.41) (end 153.035 110.49) (width 0.25) (layer B.Cu) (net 4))
 (segment (start 153.035 110.49) (end 149.225 114.3) (width 0.25) (layer F.Cu) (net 4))
 (segment (start 149.225 114.3) (end 149.225 130.175) (width 0.25) (layer B.Cu) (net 4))
 (segment (start 149.225 130.175) (end 150.02 130.97) (width 0.25) (layer B.Cu) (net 4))
 (segment (start 150.02 130.97) (end 150.02 131.525) (width 0.25) (layer B.Cu) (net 4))
 (via (at 153.035 110.49) (size 0.6) (layers F.Cu B.Cu) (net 4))
 (via (at 149.225 114.3) (size 0.6) (layers F.Cu B.Cu) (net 4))
 (segment (start 155.02 122.635) (end 154.94 122.555) (width 0.25) (layer F.Cu) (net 5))
 (segment (start 155.02 131.525) (end 155.02 122.635) (width 0.25) (layer B.Cu) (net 5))
 (segment (start 155.02 122.635) (end 154.94 122.555) (width 0.25) (layer B.Cu) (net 5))
 (segment (start 194.945 107.95) (end 163.195 107.95) (width 0.25) (layer B.Cu) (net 5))
 (segment (start 163.195 107.95) (end 160.655 110.49) (width 0.25) (layer B.Cu) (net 5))
 (segment (start 160.655 110.49) (end 156.845 114.3) (width 0.25) (layer F.Cu) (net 5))
 (segment (start 156.845 114.3) (end 154.94 116.205) (width 0.25) (layer B.Cu) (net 5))
 (segment (start 154.94 116.205) (end 154.94 122.555) (width 0.25) (layer B.Cu) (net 5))
 (via (at 160.655 110.49) (size 0.6) (layers F.Cu B.Cu) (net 5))
 (via (at 156.845 114.3) (size 0.6) (layers F.Cu B.Cu) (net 5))
 (segment (start 160.02 131.525) (end 161.845 131.525) (width 0.25) (layer B.Cu) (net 6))
 (segment (start 161.845 131.525) (end 170.815 122.555) (width 0.25) (layer B.Cu) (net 6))
 (segment (start 175.895 110.49) (end 172.085 114.3) (width 0.25) (layer F.Cu) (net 6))
 (segment (start 172.085 114.3) (end 170.815 115.57) (width 0.25) (layer B.Cu) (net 6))
 (segment (start 170.815 115.57) (end 170.815 122.555) (width 0.25) (layer B.Cu) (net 6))
 (segment (start 194.945 110.49) (end 175.895 110.49) (width 0.25) (layer B.Cu) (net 6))
 (via (at 175.895 110.49) (size 0.6) (layers F.Cu B.Cu) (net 6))
 (via (at 172.085 114.3) (size 0.6) (layers F.Cu B.Cu) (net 6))
 (segment (start 132.08 118.745) (end 132.08 105.41) (width 0.25) (layer B.Cu) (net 2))
 (segment (start 141.605 132.715) (end 132.08 123.19) (width 0.25) (layer B.Cu) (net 2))
 (segment (start 132.08 123.19) (end 132.08 118.745) (width 0.25) (layer B.Cu) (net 2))
 (segment (start 155.02 136.525) (end 153.035 136.525) (width 0.25) (layer F.Cu) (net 2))
 (segment (start 153.035 136.525) (end 150.495 133.985) (width 0.25) (layer F.Cu) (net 2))
 (segment (start 150.495 133.985) (end 142.875 133.985) (width 0.25) (layer F.Cu) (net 2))
 (segment (start 142.875 133.985) (end 141.605 132.715) (width 0.25) (layer F.Cu) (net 2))
 (segment (start 130.175 118.745) (end 132.08 118.745) (width 0.25) (layer B.Cu) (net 2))
 (via (at 141.605 132.715) (size 0.6) (layers F.Cu B.Cu) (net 2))
 (segment (start 133.985 129.54) (end 144.145 129.54) (width 0.25) (layer F.Cu) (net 16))
 (segment (start 144.145 129.54) (end 146.685 127) (width 0.25) (layer F.Cu) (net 16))
 (segment (start 146.685 127) (end 146.685 114.3) (width 0.25) (layer B.Cu) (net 16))
 (segment (start 150.495 110.49) (end 156.845 104.14) (width 0.25) (layer B.Cu) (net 16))
 (segment (start 156.845 104.14) (end 156.845 98.425) (width 0.25) (layer B.Cu) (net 16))
 (segment (start 156.845 98.425) (end 155.575 97.155) (width 0.25) (layer B.Cu) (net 16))
 (segment (start 155.575 97.155) (end 153.67 97.155) (width 0.25) (layer B.Cu) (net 16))
 (segment (start 146.685 114.3) (end 150.495 110.49) (width 0.25) (layer F.Cu) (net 16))
 (segment (start 133.985 129.54) (end 128.905 129.54) (width 0.25) (layer B.Cu) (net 16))
 (segment (start 128.905 129.54) (end 121.285 121.92) (width 0.25) (layer B.Cu) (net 16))
 (via (at 133.985 129.54) (size 0.6) (layers F.Cu B.Cu) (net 16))
 (via (at 146.685 127) (size 0.6) (layers F.Cu B.Cu) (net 16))
 (via (at 150.495 110.49) (size 0.6) (layers F.Cu B.Cu) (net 16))
 (via (at 146.685 114.3) (size 0.6) (layers F.Cu B.Cu) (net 16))
 (segment (start 127 90.17) (end 127 92.71) (width 0.25) (layer B.Cu) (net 15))
 (segment (start 127 92.71) (end 138.43 104.14) (width 0.25) (layer B.Cu) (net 15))
 (segment (start 138.43 104.14) (end 138.43 111.125) (width 0.25) (layer B.Cu) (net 15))
 (segment (start 138.43 111.125) (end 139.7 112.395) (width 0.25) (layer B.Cu) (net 15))
 (segment (start 139.7 112.395) (end 182.245 112.395) (width 0.25) (layer B.Cu) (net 15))
 (segment (start 182.245 112.395) (end 194.31 124.46) (width 0.25) (layer B.Cu) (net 15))
 (segment (start 194.31 124.46) (end 194.31 124.515) (width 0.25) (layer B.Cu) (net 15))
 (segment (start 194.945 129.54) (end 194.945 125.15) (width 0.25) (layer B.Cu) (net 15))
 (segment (start 194.945 125.15) (end 194.31 124.515) (width 0.25) (layer B.Cu) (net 15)))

